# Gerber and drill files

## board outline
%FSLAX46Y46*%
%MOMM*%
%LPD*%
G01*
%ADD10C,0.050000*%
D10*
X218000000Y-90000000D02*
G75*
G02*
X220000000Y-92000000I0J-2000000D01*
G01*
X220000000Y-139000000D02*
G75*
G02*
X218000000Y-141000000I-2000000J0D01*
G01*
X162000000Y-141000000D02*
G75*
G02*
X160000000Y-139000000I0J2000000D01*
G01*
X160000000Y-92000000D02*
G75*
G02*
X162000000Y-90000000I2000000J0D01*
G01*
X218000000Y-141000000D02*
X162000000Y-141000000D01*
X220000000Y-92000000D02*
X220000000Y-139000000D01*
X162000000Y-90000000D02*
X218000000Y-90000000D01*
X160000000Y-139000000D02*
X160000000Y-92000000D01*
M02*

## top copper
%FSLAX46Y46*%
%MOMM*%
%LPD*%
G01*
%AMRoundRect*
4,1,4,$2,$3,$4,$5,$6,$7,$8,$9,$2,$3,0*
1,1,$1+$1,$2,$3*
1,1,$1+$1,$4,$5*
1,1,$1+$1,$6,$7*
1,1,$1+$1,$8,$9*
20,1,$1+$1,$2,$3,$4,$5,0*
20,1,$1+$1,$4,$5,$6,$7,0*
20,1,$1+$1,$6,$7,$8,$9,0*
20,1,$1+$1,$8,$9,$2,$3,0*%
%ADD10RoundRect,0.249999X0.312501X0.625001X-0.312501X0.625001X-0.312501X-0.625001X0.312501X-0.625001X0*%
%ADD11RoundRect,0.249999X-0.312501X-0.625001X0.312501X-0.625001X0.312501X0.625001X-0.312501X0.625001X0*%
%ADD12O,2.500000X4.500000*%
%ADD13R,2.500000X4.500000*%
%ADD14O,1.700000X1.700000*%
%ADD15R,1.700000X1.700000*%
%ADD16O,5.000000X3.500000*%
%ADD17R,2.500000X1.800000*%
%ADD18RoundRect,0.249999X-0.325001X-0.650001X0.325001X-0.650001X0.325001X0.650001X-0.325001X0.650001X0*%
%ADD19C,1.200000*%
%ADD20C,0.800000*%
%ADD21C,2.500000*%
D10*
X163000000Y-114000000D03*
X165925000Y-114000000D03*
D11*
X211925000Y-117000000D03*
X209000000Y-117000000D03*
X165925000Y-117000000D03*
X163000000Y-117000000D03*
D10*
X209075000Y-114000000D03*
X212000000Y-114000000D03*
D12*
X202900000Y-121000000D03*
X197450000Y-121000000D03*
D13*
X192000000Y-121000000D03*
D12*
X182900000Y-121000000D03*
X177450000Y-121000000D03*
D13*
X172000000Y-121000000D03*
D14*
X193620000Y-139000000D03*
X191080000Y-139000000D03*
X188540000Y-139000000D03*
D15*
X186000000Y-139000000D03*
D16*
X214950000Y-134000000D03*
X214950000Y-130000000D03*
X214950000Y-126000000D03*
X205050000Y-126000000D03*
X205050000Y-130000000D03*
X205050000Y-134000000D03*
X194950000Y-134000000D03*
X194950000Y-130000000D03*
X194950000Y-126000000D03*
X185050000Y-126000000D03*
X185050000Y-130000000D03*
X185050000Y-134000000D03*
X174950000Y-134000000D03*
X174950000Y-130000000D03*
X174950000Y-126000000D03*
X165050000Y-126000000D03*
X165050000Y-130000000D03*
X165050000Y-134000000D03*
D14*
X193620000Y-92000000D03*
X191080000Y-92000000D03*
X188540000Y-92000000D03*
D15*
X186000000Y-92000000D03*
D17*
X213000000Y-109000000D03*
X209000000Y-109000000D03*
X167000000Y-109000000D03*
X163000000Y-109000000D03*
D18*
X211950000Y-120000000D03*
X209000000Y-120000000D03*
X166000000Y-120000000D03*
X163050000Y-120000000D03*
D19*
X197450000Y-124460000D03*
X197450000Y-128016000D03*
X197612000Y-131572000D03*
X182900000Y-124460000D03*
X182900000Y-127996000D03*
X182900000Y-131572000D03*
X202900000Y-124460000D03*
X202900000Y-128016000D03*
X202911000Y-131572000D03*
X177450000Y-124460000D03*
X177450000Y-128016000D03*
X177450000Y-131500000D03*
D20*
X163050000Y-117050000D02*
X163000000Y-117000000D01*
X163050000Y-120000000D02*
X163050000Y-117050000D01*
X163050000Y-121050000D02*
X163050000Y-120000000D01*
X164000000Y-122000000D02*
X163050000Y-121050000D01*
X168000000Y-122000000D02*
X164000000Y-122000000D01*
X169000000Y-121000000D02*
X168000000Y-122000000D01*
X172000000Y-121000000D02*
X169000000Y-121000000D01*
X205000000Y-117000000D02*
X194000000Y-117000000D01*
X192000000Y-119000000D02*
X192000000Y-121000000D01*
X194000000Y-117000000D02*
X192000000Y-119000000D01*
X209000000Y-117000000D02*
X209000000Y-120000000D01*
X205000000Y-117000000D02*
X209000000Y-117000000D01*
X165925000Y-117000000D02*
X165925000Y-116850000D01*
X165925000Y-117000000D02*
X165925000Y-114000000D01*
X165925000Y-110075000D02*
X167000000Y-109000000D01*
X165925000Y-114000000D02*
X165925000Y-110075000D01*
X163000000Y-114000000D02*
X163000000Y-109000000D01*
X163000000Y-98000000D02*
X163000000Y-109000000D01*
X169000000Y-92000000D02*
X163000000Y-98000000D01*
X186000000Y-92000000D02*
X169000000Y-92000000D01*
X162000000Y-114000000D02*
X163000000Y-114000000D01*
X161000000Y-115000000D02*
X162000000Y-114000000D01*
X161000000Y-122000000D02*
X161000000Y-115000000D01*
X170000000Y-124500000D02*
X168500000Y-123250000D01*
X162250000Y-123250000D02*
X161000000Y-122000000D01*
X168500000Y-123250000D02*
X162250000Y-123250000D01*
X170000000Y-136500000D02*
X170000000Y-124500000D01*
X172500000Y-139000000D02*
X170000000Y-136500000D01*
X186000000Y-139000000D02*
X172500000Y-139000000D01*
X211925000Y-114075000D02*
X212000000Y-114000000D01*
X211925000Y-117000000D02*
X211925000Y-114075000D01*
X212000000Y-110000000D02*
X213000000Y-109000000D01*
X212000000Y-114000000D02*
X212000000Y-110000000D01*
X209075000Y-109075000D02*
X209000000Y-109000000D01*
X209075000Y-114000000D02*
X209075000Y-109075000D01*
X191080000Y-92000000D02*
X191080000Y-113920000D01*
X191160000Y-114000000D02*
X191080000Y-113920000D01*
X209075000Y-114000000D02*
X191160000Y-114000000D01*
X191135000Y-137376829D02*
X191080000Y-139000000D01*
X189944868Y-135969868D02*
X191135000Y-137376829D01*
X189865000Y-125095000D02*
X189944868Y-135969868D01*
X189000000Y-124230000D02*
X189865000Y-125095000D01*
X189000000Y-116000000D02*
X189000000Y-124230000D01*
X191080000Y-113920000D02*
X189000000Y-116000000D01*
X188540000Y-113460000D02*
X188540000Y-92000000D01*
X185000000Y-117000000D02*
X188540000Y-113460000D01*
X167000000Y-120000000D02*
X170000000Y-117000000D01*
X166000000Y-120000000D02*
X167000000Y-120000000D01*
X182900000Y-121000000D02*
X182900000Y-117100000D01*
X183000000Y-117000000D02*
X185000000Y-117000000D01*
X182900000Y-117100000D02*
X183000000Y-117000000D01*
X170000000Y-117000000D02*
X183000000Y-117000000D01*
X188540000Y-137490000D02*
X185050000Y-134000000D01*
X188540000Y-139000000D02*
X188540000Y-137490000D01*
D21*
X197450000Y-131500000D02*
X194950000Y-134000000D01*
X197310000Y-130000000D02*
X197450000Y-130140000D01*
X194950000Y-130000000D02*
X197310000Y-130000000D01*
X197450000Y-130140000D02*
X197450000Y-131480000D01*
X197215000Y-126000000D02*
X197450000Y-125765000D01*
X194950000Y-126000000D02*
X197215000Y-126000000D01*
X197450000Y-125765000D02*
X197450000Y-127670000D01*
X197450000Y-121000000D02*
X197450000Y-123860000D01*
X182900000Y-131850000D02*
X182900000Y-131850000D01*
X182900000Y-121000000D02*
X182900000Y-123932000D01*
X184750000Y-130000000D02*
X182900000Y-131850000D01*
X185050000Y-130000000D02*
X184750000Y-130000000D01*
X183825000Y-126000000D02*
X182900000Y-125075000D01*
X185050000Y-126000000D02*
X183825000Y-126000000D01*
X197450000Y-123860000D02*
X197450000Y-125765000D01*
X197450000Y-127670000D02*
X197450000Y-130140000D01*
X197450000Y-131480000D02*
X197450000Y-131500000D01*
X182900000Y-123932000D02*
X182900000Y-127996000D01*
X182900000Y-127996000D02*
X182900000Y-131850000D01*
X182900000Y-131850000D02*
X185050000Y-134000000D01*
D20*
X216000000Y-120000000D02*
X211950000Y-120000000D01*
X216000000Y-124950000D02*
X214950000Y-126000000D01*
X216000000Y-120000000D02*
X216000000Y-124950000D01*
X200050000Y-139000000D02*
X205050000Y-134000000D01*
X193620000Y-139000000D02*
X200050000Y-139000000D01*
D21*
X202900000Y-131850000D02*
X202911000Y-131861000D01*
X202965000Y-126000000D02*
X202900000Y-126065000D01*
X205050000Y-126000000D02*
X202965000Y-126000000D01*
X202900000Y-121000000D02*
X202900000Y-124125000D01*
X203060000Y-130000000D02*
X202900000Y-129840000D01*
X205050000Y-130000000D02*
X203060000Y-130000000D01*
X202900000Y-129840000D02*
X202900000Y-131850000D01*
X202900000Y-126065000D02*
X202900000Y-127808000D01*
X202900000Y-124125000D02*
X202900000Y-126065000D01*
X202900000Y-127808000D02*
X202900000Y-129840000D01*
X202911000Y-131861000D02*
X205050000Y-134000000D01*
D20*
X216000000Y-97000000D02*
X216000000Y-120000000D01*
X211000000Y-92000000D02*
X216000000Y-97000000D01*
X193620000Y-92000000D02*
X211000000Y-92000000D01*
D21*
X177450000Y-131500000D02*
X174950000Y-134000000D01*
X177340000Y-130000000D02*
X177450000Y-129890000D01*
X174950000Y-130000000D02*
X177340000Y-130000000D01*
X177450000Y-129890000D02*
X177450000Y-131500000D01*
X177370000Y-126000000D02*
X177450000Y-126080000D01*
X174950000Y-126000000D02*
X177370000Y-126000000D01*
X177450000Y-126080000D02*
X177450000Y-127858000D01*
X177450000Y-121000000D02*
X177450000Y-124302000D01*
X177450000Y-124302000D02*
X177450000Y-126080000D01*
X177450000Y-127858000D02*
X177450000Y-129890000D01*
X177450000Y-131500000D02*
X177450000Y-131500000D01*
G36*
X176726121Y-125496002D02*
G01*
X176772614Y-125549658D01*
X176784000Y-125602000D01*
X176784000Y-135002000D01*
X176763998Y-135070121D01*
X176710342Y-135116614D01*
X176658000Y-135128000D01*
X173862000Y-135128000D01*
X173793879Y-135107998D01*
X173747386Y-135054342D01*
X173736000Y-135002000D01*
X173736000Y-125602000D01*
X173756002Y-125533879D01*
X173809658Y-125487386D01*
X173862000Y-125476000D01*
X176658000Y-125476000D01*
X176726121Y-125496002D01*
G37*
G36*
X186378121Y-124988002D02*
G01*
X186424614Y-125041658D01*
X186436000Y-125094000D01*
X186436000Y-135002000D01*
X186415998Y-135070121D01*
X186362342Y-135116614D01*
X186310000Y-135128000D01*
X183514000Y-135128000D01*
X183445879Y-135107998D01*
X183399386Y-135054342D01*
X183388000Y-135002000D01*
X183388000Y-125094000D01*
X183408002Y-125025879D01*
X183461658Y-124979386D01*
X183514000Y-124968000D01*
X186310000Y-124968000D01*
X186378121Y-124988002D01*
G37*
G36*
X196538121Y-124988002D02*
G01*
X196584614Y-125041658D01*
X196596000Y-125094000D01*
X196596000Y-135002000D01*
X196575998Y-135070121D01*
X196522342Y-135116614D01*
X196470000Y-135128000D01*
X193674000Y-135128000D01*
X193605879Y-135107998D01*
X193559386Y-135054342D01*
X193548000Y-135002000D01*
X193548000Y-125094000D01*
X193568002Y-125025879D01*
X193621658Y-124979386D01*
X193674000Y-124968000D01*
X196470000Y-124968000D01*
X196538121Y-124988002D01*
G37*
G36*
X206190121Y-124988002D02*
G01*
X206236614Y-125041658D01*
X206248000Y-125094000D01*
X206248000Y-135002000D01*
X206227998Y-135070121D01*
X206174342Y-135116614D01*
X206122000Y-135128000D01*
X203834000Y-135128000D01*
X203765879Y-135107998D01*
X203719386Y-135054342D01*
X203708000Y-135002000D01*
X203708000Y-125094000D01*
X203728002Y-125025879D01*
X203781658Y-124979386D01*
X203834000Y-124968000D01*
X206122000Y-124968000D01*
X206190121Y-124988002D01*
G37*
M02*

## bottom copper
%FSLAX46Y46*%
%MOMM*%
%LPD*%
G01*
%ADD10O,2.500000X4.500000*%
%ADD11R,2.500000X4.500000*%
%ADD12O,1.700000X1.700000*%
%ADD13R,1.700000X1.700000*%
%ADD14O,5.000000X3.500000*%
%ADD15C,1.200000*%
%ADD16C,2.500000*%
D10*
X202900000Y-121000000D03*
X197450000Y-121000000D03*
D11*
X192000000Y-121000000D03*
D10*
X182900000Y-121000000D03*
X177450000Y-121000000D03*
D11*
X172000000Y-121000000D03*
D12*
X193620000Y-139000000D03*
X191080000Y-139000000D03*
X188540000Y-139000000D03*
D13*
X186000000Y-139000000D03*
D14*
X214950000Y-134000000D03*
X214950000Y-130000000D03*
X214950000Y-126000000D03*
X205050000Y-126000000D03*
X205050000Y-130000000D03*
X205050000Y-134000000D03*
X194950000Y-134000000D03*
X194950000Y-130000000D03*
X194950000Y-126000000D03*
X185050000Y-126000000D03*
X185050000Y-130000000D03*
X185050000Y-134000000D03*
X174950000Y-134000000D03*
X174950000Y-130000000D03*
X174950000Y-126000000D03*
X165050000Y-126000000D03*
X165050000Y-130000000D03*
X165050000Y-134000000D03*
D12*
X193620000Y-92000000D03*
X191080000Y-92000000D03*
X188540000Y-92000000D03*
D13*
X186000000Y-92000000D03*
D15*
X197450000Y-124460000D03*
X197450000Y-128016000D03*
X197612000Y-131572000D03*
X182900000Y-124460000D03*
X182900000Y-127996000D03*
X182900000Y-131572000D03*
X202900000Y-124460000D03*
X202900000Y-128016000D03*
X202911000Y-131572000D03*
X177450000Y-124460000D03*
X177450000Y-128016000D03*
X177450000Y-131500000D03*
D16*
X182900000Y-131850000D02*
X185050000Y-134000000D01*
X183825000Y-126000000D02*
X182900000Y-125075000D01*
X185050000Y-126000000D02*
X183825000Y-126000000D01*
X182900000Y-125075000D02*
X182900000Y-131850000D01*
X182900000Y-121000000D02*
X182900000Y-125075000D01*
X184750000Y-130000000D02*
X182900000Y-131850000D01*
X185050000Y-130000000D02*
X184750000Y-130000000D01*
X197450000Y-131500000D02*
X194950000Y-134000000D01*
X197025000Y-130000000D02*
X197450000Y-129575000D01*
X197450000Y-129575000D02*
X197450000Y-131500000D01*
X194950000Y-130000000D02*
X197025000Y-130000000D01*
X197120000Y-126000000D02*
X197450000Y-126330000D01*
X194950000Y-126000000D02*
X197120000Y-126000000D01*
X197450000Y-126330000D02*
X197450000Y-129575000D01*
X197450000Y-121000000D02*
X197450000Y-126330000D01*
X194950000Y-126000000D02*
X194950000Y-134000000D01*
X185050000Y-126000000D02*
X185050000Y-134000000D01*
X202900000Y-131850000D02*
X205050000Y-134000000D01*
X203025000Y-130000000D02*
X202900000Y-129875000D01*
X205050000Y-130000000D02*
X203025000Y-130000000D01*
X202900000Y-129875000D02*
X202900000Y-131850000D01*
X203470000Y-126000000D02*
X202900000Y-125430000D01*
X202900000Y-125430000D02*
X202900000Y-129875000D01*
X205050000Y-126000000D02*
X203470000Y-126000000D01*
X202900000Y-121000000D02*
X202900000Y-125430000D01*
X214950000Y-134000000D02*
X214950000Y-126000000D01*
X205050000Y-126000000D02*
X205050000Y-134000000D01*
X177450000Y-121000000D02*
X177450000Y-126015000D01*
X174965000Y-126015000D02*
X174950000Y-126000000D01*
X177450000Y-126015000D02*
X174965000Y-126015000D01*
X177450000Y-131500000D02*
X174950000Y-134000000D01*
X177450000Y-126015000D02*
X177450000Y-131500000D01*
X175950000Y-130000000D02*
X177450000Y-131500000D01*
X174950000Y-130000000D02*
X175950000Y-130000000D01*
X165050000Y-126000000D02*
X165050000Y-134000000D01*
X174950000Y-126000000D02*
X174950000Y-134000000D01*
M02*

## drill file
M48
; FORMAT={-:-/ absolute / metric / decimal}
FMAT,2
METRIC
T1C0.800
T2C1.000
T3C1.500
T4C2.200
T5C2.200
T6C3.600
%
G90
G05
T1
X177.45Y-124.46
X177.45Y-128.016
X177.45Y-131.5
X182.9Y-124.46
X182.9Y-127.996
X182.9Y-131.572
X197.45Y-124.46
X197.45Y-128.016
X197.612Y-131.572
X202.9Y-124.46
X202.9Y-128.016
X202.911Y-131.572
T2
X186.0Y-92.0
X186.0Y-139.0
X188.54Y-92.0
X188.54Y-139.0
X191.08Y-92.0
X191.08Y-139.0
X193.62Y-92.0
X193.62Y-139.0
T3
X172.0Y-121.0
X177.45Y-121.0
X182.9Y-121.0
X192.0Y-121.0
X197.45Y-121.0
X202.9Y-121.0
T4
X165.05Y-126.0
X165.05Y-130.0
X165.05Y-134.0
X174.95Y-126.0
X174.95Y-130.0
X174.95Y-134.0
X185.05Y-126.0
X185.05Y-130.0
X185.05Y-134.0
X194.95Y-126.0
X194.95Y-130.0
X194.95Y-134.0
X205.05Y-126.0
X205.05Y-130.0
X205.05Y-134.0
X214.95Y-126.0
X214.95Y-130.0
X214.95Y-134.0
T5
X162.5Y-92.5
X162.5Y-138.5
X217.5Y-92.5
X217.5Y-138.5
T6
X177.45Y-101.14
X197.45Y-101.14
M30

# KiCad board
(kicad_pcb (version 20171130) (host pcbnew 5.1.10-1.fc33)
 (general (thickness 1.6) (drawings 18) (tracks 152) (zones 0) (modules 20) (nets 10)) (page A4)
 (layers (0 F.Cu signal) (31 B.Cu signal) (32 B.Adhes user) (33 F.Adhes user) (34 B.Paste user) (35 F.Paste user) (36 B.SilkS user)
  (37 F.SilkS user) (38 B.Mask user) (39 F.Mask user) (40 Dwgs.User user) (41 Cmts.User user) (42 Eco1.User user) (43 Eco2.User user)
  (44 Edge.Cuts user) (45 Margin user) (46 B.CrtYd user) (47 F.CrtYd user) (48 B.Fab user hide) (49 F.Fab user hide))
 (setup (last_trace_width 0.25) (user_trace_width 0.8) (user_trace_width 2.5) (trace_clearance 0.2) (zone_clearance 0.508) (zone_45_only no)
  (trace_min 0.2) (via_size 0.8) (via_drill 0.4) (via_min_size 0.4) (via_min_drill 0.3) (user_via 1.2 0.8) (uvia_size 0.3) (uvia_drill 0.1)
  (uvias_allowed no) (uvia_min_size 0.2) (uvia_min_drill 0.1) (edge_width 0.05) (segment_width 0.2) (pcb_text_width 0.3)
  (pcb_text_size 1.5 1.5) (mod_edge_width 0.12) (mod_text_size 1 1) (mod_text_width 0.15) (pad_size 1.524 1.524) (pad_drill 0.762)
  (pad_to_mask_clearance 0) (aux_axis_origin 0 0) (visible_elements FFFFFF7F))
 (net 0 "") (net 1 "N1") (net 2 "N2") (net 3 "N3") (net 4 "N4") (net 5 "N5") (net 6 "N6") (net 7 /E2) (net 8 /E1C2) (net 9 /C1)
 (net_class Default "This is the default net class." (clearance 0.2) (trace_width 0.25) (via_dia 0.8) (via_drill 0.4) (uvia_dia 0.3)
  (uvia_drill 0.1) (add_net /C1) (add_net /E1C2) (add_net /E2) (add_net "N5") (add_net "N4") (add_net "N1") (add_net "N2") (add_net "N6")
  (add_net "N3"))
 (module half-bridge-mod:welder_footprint (layer F.Cu) (at 178.5 110.7)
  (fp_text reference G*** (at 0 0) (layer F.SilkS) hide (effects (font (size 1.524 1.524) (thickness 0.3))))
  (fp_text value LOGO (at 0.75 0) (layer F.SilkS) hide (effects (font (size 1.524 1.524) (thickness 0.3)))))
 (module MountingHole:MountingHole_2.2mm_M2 (layer F.Cu) (at 162.5 138.5)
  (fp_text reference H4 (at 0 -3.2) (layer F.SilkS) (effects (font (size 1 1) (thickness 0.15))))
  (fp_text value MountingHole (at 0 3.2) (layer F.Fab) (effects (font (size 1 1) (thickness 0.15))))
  (pad 1 np_thru_hole circle (at 0 0) (size 2.2 2.2) (drill 2.2) (layers *.Cu *.Mask)))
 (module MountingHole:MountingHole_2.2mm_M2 (layer F.Cu) (at 217.5 138.5)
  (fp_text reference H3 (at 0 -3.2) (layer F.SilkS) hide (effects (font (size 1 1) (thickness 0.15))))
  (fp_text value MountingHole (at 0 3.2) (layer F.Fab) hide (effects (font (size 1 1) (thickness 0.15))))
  (pad 1 np_thru_hole circle (at 0 0) (size 2.2 2.2) (drill 2.2) (layers *.Cu *.Mask)))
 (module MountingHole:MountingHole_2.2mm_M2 (layer F.Cu) (at 162.5 92.5)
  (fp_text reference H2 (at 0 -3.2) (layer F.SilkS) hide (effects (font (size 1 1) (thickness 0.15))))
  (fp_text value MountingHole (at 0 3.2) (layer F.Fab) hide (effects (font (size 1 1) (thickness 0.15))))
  (pad 1 np_thru_hole circle (at 0 0) (size 2.2 2.2) (drill 2.2) (layers *.Cu *.Mask)))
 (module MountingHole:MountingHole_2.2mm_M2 (layer F.Cu) (at 217.5 92.5)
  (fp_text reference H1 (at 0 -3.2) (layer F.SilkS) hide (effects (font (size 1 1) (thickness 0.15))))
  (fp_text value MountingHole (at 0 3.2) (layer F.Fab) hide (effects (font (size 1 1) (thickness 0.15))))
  (pad 1 np_thru_hole circle (at 0 0) (size 2.2 2.2) (drill 2.2) (layers *.Cu *.Mask)))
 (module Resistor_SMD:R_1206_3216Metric (layer F.Cu) (at 164.4625 114 180)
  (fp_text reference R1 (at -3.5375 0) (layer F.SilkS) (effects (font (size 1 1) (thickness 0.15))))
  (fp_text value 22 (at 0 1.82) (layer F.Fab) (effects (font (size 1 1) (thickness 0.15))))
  (pad 2 smd roundrect (at 1.4625 0 180) (size 1.125 1.75) (layers F.Cu F.Paste F.Mask) (roundrect_rratio 0.2222213333333333) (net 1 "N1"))
  (pad 1 smd roundrect (at -1.4625 0 180) (size 1.125 1.75) (layers F.Cu F.Paste F.Mask) (roundrect_rratio 0.2222213333333333) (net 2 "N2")))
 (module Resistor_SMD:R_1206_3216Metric (layer F.Cu) (at 210.4625 117)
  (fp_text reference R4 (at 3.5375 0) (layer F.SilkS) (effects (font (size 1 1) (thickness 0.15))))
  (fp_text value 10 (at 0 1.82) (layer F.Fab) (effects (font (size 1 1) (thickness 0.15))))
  (pad 2 smd roundrect (at 1.4625 0) (size 1.125 1.75) (layers F.Cu F.Paste F.Mask) (roundrect_rratio 0.2222213333333333) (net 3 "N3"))
  (pad 1 smd roundrect (at -1.4625 0) (size 1.125 1.75) (layers F.Cu F.Paste F.Mask) (roundrect_rratio 0.2222213333333333) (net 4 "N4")))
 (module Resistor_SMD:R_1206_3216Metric (layer F.Cu) (at 164.4625 117)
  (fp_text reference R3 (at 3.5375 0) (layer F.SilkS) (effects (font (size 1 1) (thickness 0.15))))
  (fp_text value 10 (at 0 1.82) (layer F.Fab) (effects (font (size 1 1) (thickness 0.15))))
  (pad 2 smd roundrect (at 1.4625 0) (size 1.125 1.75) (layers F.Cu F.Paste F.Mask) (roundrect_rratio 0.2222213333333333) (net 2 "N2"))
  (pad 1 smd roundrect (at -1.4625 0) (size 1.125 1.75) (layers F.Cu F.Paste F.Mask) (roundrect_rratio 0.2222213333333333) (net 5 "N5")))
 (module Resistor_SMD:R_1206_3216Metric (layer F.Cu) (at 210.5375 114 180)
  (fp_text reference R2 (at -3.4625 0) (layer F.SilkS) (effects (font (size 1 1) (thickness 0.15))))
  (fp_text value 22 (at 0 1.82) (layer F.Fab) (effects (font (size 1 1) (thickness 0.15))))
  (pad 2 smd roundrect (at 1.4625 0 180) (size 1.125 1.75) (layers F.Cu F.Paste F.Mask) (roundrect_rratio 0.2222213333333333) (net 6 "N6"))
  (pad 1 smd roundrect (at -1.4625 0 180) (size 1.125 1.75) (layers F.Cu F.Paste F.Mask) (roundrect_rratio 0.2222213333333333) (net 3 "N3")))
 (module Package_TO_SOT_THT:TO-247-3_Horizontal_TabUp (layer B.Cu) (at 192 121)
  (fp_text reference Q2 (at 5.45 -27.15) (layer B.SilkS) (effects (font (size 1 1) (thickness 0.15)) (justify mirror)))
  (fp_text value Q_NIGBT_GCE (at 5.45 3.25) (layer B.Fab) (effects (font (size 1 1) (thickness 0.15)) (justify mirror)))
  (pad 3 thru_hole oval (at 10.9 0) (size 2.5 4.5) (drill 1.5) (layers *.Cu *.Mask) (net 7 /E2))
  (pad 2 thru_hole oval (at 5.45 0) (size 2.5 4.5) (drill 1.5) (layers *.Cu *.Mask) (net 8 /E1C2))
  (pad 1 thru_hole rect (at 0 0) (size 2.5 4.5) (drill 1.5) (layers *.Cu *.Mask) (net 4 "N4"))
  (pad "" np_thru_hole oval (at 5.45 -19.86) (size 3.6 3.6) (drill 3.6) (layers *.Cu *.Mask)))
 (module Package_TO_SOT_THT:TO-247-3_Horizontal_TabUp (layer B.Cu) (at 172 121)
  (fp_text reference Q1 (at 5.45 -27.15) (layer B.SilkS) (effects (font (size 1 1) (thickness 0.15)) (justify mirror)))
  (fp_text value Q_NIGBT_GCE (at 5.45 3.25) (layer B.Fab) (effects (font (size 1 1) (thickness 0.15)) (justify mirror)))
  (pad 3 thru_hole oval (at 10.9 0) (size 2.5 4.5) (drill 1.5) (layers *.Cu *.Mask) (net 8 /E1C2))
  (pad 2 thru_hole oval (at 5.45 0) (size 2.5 4.5) (drill 1.5) (layers *.Cu *.Mask) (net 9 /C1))
  (pad 1 thru_hole rect (at 0 0) (size 2.5 4.5) (drill 1.5) (layers *.Cu *.Mask) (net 5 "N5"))
  (pad "" np_thru_hole oval (at 5.45 -19.86) (size 3.6 3.6) (drill 3.6) (layers *.Cu *.Mask)))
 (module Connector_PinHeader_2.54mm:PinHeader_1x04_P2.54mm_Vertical (layer F.Cu) (at 186 139 90)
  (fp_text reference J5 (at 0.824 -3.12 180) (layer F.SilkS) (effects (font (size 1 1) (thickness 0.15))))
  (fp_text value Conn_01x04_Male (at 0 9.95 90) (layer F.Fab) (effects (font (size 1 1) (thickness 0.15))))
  (pad 4 thru_hole oval (at 0 7.62 90) (size 1.7 1.7) (drill 1) (layers *.Cu *.Mask) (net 7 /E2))
  (pad 3 thru_hole oval (at 0 5.08 90) (size 1.7 1.7) (drill 1) (layers *.Cu *.Mask) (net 6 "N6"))
  (pad 2 thru_hole oval (at 0 2.54 90) (size 1.7 1.7) (drill 1) (layers *.Cu *.Mask) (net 8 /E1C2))
  (pad 1 thru_hole rect (at 0 0 90) (size 1.7 1.7) (drill 1) (layers *.Cu *.Mask) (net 1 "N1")))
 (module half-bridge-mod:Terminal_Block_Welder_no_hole (layer F.Cu) (at 210 130 90)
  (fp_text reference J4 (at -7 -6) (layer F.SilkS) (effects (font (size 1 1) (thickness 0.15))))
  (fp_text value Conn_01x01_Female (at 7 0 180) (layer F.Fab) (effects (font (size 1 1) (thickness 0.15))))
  (pad 1 thru_hole oval (at -4 4.95 180) (size 5 3.5) (drill 2.2) (layers *.Cu *.Mask) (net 7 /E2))
  (pad 1 thru_hole oval (at 0 4.95 180) (size 5 3.5) (drill 2.2) (layers *.Cu *.Mask) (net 7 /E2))
  (pad 1 thru_hole oval (at 4 4.95 180) (size 5 3.5) (drill 2.2) (layers *.Cu *.Mask) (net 7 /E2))
  (pad 1 thru_hole oval (at 4 -4.95 180) (size 5 3.5) (drill 2.2) (layers *.Cu *.Mask) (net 7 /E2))
  (pad 1 thru_hole oval (at 0 -4.95 180) (size 5 3.5) (drill 2.2) (layers *.Cu *.Mask) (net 7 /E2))
  (pad 1 thru_hole oval (at -4 -4.95 180) (size 5 3.5) (drill 2.2) (layers *.Cu *.Mask) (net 7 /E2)))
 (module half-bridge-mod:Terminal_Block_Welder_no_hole (layer F.Cu) (at 190 130 90)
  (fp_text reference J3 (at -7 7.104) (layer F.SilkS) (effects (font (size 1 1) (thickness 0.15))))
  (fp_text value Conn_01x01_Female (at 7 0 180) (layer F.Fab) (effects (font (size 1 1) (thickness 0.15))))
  (pad 1 thru_hole oval (at -4 4.95 180) (size 5 3.5) (drill 2.2) (layers *.Cu *.Mask) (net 8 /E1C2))
  (pad 1 thru_hole oval (at 0 4.95 180) (size 5 3.5) (drill 2.2) (layers *.Cu *.Mask) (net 8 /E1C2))
  (pad 1 thru_hole oval (at 4 4.95 180) (size 5 3.5) (drill 2.2) (layers *.Cu *.Mask) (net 8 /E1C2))
  (pad 1 thru_hole oval (at 4 -4.95 180) (size 5 3.5) (drill 2.2) (layers *.Cu *.Mask) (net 8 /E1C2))
  (pad 1 thru_hole oval (at 0 -4.95 180) (size 5 3.5) (drill 2.2) (layers *.Cu *.Mask) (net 8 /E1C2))
  (pad 1 thru_hole oval (at -4 -4.95 180) (size 5 3.5) (drill 2.2) (layers *.Cu *.Mask) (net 8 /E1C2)))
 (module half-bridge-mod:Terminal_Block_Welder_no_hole (layer F.Cu) (at 170 130 90)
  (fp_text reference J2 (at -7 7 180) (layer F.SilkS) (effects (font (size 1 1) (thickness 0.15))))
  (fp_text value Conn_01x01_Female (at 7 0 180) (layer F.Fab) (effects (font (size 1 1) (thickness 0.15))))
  (pad 1 thru_hole oval (at -4 4.95 180) (size 5 3.5) (drill 2.2) (layers *.Cu *.Mask) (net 9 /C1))
  (pad 1 thru_hole oval (at 0 4.95 180) (size 5 3.5) (drill 2.2) (layers *.Cu *.Mask) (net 9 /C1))
  (pad 1 thru_hole oval (at 4 4.95 180) (size 5 3.5) (drill 2.2) (layers *.Cu *.Mask) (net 9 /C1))
  (pad 1 thru_hole oval (at 4 -4.95 180) (size 5 3.5) (drill 2.2) (layers *.Cu *.Mask) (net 9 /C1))
  (pad 1 thru_hole oval (at 0 -4.95 180) (size 5 3.5) (drill 2.2) (layers *.Cu *.Mask) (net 9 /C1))
  (pad 1 thru_hole oval (at -4 -4.95 180) (size 5 3.5) (drill 2.2) (layers *.Cu *.Mask) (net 9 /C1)))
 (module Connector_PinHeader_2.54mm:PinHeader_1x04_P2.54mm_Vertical (layer F.Cu) (at 186 92 90)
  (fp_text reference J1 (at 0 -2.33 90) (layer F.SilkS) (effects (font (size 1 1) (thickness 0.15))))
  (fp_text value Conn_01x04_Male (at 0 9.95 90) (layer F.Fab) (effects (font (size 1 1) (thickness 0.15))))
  (pad 4 thru_hole oval (at 0 7.62 90) (size 1.7 1.7) (drill 1) (layers *.Cu *.Mask) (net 7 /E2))
  (pad 3 thru_hole oval (at 0 5.08 90) (size 1.7 1.7) (drill 1) (layers *.Cu *.Mask) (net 6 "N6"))
  (pad 2 thru_hole oval (at 0 2.54 90) (size 1.7 1.7) (drill 1) (layers *.Cu *.Mask) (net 8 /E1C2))
  (pad 1 thru_hole rect (at 0 0 90) (size 1.7 1.7) (drill 1) (layers *.Cu *.Mask) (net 1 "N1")))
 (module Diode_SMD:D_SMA (layer F.Cu) (at 211 109)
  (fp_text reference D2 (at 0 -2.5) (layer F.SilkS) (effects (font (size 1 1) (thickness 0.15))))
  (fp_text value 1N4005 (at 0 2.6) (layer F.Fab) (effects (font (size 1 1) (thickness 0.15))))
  (pad 2 smd rect (at 2 0) (size 2.5 1.8) (layers F.Cu F.Paste F.Mask) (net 3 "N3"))
  (pad 1 smd rect (at -2 0) (size 2.5 1.8) (layers F.Cu F.Paste F.Mask) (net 6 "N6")))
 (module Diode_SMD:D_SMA (layer F.Cu) (at 165 109)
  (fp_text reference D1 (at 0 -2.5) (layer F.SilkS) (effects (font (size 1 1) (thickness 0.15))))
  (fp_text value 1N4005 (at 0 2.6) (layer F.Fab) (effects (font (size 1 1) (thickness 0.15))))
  (pad 2 smd rect (at 2 0) (size 2.5 1.8) (layers F.Cu F.Paste F.Mask) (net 2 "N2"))
  (pad 1 smd rect (at -2 0) (size 2.5 1.8) (layers F.Cu F.Paste F.Mask) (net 1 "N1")))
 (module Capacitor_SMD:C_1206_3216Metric (layer F.Cu) (at 210.475 120)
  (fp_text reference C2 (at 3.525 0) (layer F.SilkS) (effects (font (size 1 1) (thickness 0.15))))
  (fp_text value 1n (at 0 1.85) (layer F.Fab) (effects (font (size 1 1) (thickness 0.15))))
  (pad 2 smd roundrect (at 1.475 0) (size 1.15 1.8) (layers F.Cu F.Paste F.Mask) (roundrect_rratio 0.2173904347826087) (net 7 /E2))
  (pad 1 smd roundrect (at -1.475 0) (size 1.15 1.8) (layers F.Cu F.Paste F.Mask) (roundrect_rratio 0.2173904347826087) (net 4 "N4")))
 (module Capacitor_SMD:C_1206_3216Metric (layer F.Cu) (at 164.525 120)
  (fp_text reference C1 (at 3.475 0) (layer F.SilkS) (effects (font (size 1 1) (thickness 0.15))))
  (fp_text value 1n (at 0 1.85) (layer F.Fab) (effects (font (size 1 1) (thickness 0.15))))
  (pad 2 smd roundrect (at 1.475 0) (size 1.15 1.8) (layers F.Cu F.Paste F.Mask) (roundrect_rratio 0.2173904347826087) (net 8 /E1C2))
  (pad 1 smd roundrect (at -1.475 0) (size 1.15 1.8) (layers F.Cu F.Paste F.Mask) (roundrect_rratio 0.2173904347826087) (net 5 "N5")))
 (gr_arc (start 218 92) (end 220 92) (angle -90) (layer Edge.Cuts) (width 0.05))
 (gr_arc (start 218 139) (end 218 141) (angle -90) (layer Edge.Cuts) (width 0.05))
 (gr_arc (start 162 139) (end 160 139) (angle -90) (layer Edge.Cuts) (width 0.05))
 (gr_arc (start 162 92) (end 162 90) (angle -90) (layer Edge.Cuts) (width 0.05))
 (gr_line (start 218 141) (end 162 141) (layer Edge.Cuts) (width 0.05))
 (gr_line (start 220 92) (end 220 139) (layer Edge.Cuts) (width 0.05))
 (gr_line (start 162 90) (end 218 90) (layer Edge.Cuts) (width 0.05))
 (gr_line (start 160 139) (end 160 92) (layer Edge.Cuts) (width 0.05))
 (segment (start 163.05 117.05) (end 163 117) (width 0.8) (layer F.Cu) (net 5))
 (segment (start 163.05 120) (end 163.05 117.05) (width 0.8) (layer F.Cu) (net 5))
 (segment (start 163.05 121.05) (end 163.05 120) (width 0.8) (layer F.Cu) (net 5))
 (segment (start 164 122) (end 163.05 121.05) (width 0.8) (layer F.Cu) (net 5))
 (segment (start 168 122) (end 164 122) (width 0.8) (layer F.Cu) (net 5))
 (segment (start 169 121) (end 168 122) (width 0.8) (layer F.Cu) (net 5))
 (segment (start 172 121) (end 169 121) (width 0.8) (layer F.Cu) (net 5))
 (segment (start 205 117) (end 194 117) (width 0.8) (layer F.Cu) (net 4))
 (segment (start 192 119) (end 192 121) (width 0.8) (layer F.Cu) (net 4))
 (segment (start 194 117) (end 192 119) (width 0.8) (layer F.Cu) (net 4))
 (segment (start 209 117) (end 209 120) (width 0.8) (layer F.Cu) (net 4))
 (segment (start 205 117) (end 209 117) (width 0.8) (layer F.Cu) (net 4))
 (segment (start 165.925 117) (end 165.925 116.85) (width 0.8) (layer F.Cu) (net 2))
 (segment (start 165.925 117) (end 165.925 114) (width 0.8) (layer F.Cu) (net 2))
 (segment (start 165.925 110.075) (end 167 109) (width 0.8) (layer F.Cu) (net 2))
 (segment (start 165.925 114) (end 165.925 110.075) (width 0.8) (layer F.Cu) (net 2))
 (segment (start 163 114) (end 163 109) (width 0.8) (layer F.Cu) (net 1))
 (segment (start 163 98) (end 163 109) (width 0.8) (layer F.Cu) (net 1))
 (segment (start 169 92) (end 163 98) (width 0.8) (layer F.Cu) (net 1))
 (segment (start 186 92) (end 169 92) (width 0.8) (layer F.Cu) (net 1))
 (segment (start 162 114) (end 163 114) (width 0.8) (layer F.Cu) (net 1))
 (segment (start 161 115) (end 162 114) (width 0.8) (layer F.Cu) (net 1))
 (segment (start 161 122) (end 161 115) (width 0.8) (layer F.Cu) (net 1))
 (segment (start 170 124.5) (end 168.5 123.25) (width 0.8) (layer F.Cu) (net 1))
 (segment (start 162.25 123.25) (end 161 122) (width 0.8) (layer F.Cu) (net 1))
 (segment (start 168.5 123.25) (end 162.25 123.25) (width 0.8) (layer F.Cu) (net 1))
 (segment (start 170 136.5) (end 170 124.5) (width 0.8) (layer F.Cu) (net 1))
 (segment (start 172.5 139) (end 170 136.5) (width 0.8) (layer F.Cu) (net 1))
 (segment (start 186 139) (end 172.5 139) (width 0.8) (layer F.Cu) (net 1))
 (segment (start 211.925 114.075) (end 212 114) (width 0.8) (layer F.Cu) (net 3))
 (segment (start 211.925 117) (end 211.925 114.075) (width 0.8) (layer F.Cu) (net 3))
 (segment (start 212 110) (end 213 109) (width 0.8) (layer F.Cu) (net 3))
 (segment (start 212 114) (end 212 110) (width 0.8) (layer F.Cu) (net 3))
 (segment (start 209.075 109.075) (end 209 109) (width 0.8) (layer F.Cu) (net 6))
 (segment (start 209.075 114) (end 209.075 109.075) (width 0.8) (layer F.Cu) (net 6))
 (segment (start 191.08 92) (end 191.08 113.92) (width 0.8) (layer F.Cu) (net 6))
 (segment (start 191.16 114) (end 191.08 113.92) (width 0.8) (layer F.Cu) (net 6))
 (segment (start 209.075 114) (end 191.16 114) (width 0.8) (layer F.Cu) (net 6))
 (segment (start 191.135 137.376829) (end 191.08 139) (width 0.8) (layer F.Cu) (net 6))
 (segment (start 189.944868 135.969868) (end 191.135 137.376829) (width 0.8) (layer F.Cu) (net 6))
 (segment (start 189.865 125.095) (end 189.944868 135.969868) (width 0.8) (layer F.Cu) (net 6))
 (segment (start 189 124.23) (end 189.865 125.095) (width 0.8) (layer F.Cu) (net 6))
 (segment (start 189 116) (end 189 124.23) (width 0.8) (layer F.Cu) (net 6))
 (segment (start 191.08 113.92) (end 189 116) (width 0.8) (layer F.Cu) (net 6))
 (segment (start 188.54 113.46) (end 188.54 92) (width 0.8) (layer F.Cu) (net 8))
 (segment (start 185 117) (end 188.54 113.46) (width 0.8) (layer F.Cu) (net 8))
 (segment (start 167 120) (end 170 117) (width 0.8) (layer F.Cu) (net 8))
 (segment (start 166 120) (end 167 120) (width 0.8) (layer F.Cu) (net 8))
 (segment (start 182.9 121) (end 182.9 117.1) (width 0.8) (layer F.Cu) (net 8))
 (segment (start 183 117) (end 185 117) (width 0.8) (layer F.Cu) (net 8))
 (segment (start 182.9 117.1) (end 183 117) (width 0.8) (layer F.Cu) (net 8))
 (segment (start 170 117) (end 183 117) (width 0.8) (layer F.Cu) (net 8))
 (segment (start 188.54 137.49) (end 185.05 134) (width 0.8) (layer F.Cu) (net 8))
 (segment (start 188.54 139) (end 188.54 137.49) (width 0.8) (layer F.Cu) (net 8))
 (segment (start 182.9 131.85) (end 185.05 134) (width 2.5) (layer B.Cu) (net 8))
 (segment (start 183.825 126) (end 182.9 125.075) (width 2.5) (layer B.Cu) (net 8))
 (segment (start 185.05 126) (end 183.825 126) (width 2.5) (layer B.Cu) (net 8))
 (segment (start 182.9 125.075) (end 182.9 131.85) (width 2.5) (layer B.Cu) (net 8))
 (segment (start 182.9 121) (end 182.9 125.075) (width 2.5) (layer B.Cu) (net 8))
 (segment (start 184.75 130) (end 182.9 131.85) (width 2.5) (layer B.Cu) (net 8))
 (segment (start 185.05 130) (end 184.75 130) (width 2.5) (layer B.Cu) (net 8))
 (segment (start 197.45 131.5) (end 194.95 134) (width 2.5) (layer B.Cu) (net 8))
 (segment (start 197.025 130) (end 197.45 129.575) (width 2.5) (layer B.Cu) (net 8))
 (segment (start 197.45 129.575) (end 197.45 131.5) (width 2.5) (layer B.Cu) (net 8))
 (segment (start 194.95 130) (end 197.025 130) (width 2.5) (layer B.Cu) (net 8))
 (segment (start 197.12 126) (end 197.45 126.33) (width 2.5) (layer B.Cu) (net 8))
 (segment (start 194.95 126) (end 197.12 126) (width 2.5) (layer B.Cu) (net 8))
 (segment (start 197.45 126.33) (end 197.45 129.575) (width 2.5) (layer B.Cu) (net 8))
 (segment (start 197.45 121) (end 197.45 126.33) (width 2.5) (layer B.Cu) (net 8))
 (segment (start 197.45 131.5) (end 194.95 134) (width 2.5) (layer F.Cu) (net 8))
 (segment (start 197.31 130) (end 197.45 130.14) (width 2.5) (layer F.Cu) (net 8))
 (segment (start 194.95 130) (end 197.31 130) (width 2.5) (layer F.Cu) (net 8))
 (segment (start 197.45 130.14) (end 197.45 131.48) (width 2.5) (layer F.Cu) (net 8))
 (segment (start 197.215 126) (end 197.45 125.765) (width 2.5) (layer F.Cu) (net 8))
 (segment (start 194.95 126) (end 197.215 126) (width 2.5) (layer F.Cu) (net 8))
 (segment (start 197.45 125.765) (end 197.45 127.67) (width 2.5) (layer F.Cu) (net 8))
 (segment (start 197.45 121) (end 197.45 123.86) (width 2.5) (layer F.Cu) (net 8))
 (segment (start 182.9 131.85) (end 182.9 131.85) (width 2.5) (layer F.Cu) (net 8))
 (segment (start 182.9 121) (end 182.9 123.932) (width 2.5) (layer F.Cu) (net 8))
 (segment (start 184.75 130) (end 182.9 131.85) (width 2.5) (layer F.Cu) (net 8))
 (segment (start 185.05 130) (end 184.75 130) (width 2.5) (layer F.Cu) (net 8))
 (segment (start 183.825 126) (end 182.9 125.075) (width 2.5) (layer F.Cu) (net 8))
 (segment (start 185.05 126) (end 183.825 126) (width 2.5) (layer F.Cu) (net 8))
 (segment (start 194.95 126) (end 194.95 134) (width 2.5) (layer B.Cu) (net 8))
 (segment (start 185.05 126) (end 185.05 134) (width 2.5) (layer B.Cu) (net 8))
 (segment (start 197.45 123.86) (end 197.45 125.765) (width 2.5) (layer F.Cu) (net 8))
 (via (at 197.45 124.46) (size 1.2) (drill 0.8) (layers F.Cu B.Cu) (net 8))
 (segment (start 197.45 127.67) (end 197.45 130.14) (width 2.5) (layer F.Cu) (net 8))
 (via (at 197.45 128.016) (size 1.2) (drill 0.8) (layers F.Cu B.Cu) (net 8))
 (segment (start 197.45 131.48) (end 197.45 131.5) (width 2.5) (layer F.Cu) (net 8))
 (via (at 197.612 131.572) (size 1.2) (drill 0.8) (layers F.Cu B.Cu) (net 8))
 (segment (start 182.9 123.932) (end 182.9 127.996) (width 2.5) (layer F.Cu) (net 8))
 (via (at 182.9 124.46) (size 1.2) (drill 0.8) (layers F.Cu B.Cu) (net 8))
 (segment (start 182.9 127.996) (end 182.9 131.85) (width 2.5) (layer F.Cu) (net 8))
 (via (at 182.9 127.996) (size 1.2) (drill 0.8) (layers F.Cu B.Cu) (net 8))
 (segment (start 182.9 131.85) (end 185.05 134) (width 2.5) (layer F.Cu) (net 8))
 (via (at 182.9 131.572) (size 1.2) (drill 0.8) (layers F.Cu B.Cu) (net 8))
 (segment (start 216 120) (end 211.95 120) (width 0.8) (layer F.Cu) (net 7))
 (segment (start 216 124.95) (end 214.95 126) (width 0.8) (layer F.Cu) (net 7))
 (segment (start 216 120) (end 216 124.95) (width 0.8) (layer F.Cu) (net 7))
 (segment (start 200.05 139) (end 205.05 134) (width 0.8) (layer F.Cu) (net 7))
 (segment (start 193.62 139) (end 200.05 139) (width 0.8) (layer F.Cu) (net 7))
 (segment (start 202.9 131.85) (end 205.05 134) (width 2.5) (layer B.Cu) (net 7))
 (segment (start 203.025 130) (end 202.9 129.875) (width 2.5) (layer B.Cu) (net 7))
 (segment (start 205.05 130) (end 203.025 130) (width 2.5) (layer B.Cu) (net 7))
 (segment (start 202.9 129.875) (end 202.9 131.85) (width 2.5) (layer B.Cu) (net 7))
 (segment (start 203.47 126) (end 202.9 125.43) (width 2.5) (layer B.Cu) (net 7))
 (segment (start 202.9 125.43) (end 202.9 129.875) (width 2.5) (layer B.Cu) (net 7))
 (segment (start 205.05 126) (end 203.47 126) (width 2.5) (layer B.Cu) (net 7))
 (segment (start 202.9 121) (end 202.9 125.43) (width 2.5) (layer B.Cu) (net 7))
 (segment (start 202.9 131.85) (end 202.911 131.861) (width 2.5) (layer F.Cu) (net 7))
 (segment (start 202.965 126) (end 202.9 126.065) (width 2.5) (layer F.Cu) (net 7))
 (segment (start 205.05 126) (end 202.965 126) (width 2.5) (layer F.Cu) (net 7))
 (segment (start 202.9 121) (end 202.9 124.125) (width 2.5) (layer F.Cu) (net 7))
 (segment (start 203.06 130) (end 202.9 129.84) (width 2.5) (layer F.Cu) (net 7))
 (segment (start 205.05 130) (end 203.06 130) (width 2.5) (layer F.Cu) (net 7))
 (segment (start 202.9 129.84) (end 202.9 131.85) (width 2.5) (layer F.Cu) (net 7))
 (segment (start 202.9 126.065) (end 202.9 127.808) (width 2.5) (layer F.Cu) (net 7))
 (segment (start 214.95 134) (end 214.95 126) (width 2.5) (layer B.Cu) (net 7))
 (segment (start 205.05 126) (end 205.05 134) (width 2.5) (layer B.Cu) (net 7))
 (segment (start 202.9 124.125) (end 202.9 126.065) (width 2.5) (layer F.Cu) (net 7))
 (via (at 202.9 124.46) (size 1.2) (drill 0.8) (layers F.Cu B.Cu) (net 7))
 (segment (start 202.9 127.808) (end 202.9 129.84) (width 2.5) (layer F.Cu) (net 7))
 (via (at 202.9 128.016) (size 1.2) (drill 0.8) (layers F.Cu B.Cu) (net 7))
 (segment (start 202.911 131.861) (end 205.05 134) (width 2.5) (layer F.Cu) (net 7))
 (via (at 202.911 131.572) (size 1.2) (drill 0.8) (layers F.Cu B.Cu) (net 7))
 (segment (start 216 97) (end 216 120) (width 0.8) (layer F.Cu) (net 7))
 (segment (start 211 92) (end 216 97) (width 0.8) (layer F.Cu) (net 7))
 (segment (start 193.62 92) (end 211 92) (width 0.8) (layer F.Cu) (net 7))
 (segment (start 177.45 121) (end 177.45 126.015) (width 2.5) (layer B.Cu) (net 9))
 (segment (start 174.965 126.015) (end 174.95 126) (width 2.5) (layer B.Cu) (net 9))
 (segment (start 177.45 126.015) (end 174.965 126.015) (width 2.5) (layer B.Cu) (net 9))
 (segment (start 177.45 131.5) (end 174.95 134) (width 2.5) (layer B.Cu) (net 9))
 (segment (start 177.45 126.015) (end 177.45 131.5) (width 2.5) (layer B.Cu) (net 9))
 (segment (start 175.95 130) (end 177.45 131.5) (width 2.5) (layer B.Cu) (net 9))
 (segment (start 174.95 130) (end 175.95 130) (width 2.5) (layer B.Cu) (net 9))
 (segment (start 165.05 126) (end 165.05 134) (width 2.5) (layer B.Cu) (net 9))
 (segment (start 177.45 131.5) (end 174.95 134) (width 2.5) (layer F.Cu) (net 9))
 (segment (start 177.34 130) (end 177.45 129.89) (width 2.5) (layer F.Cu) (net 9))
 (segment (start 174.95 130) (end 177.34 130) (width 2.5) (layer F.Cu) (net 9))
 (segment (start 177.45 129.89) (end 177.45 131.5) (width 2.5) (layer F.Cu) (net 9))
 (segment (start 177.37 126) (end 177.45 126.08) (width 2.5) (layer F.Cu) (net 9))
 (segment (start 174.95 126) (end 177.37 126) (width 2.5) (layer F.Cu) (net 9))
 (segment (start 177.45 126.08) (end 177.45 127.858) (width 2.5) (layer F.Cu) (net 9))
 (segment (start 177.45 121) (end 177.45 124.302) (width 2.5) (layer F.Cu) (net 9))
 (segment (start 174.95 126) (end 174.95 134) (width 2.5) (layer B.Cu) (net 9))
 (segment (start 177.45 124.302) (end 177.45 126.08) (width 2.5) (layer F.Cu) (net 9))
 (via (at 177.45 124.46) (size 1.2) (drill 0.8) (layers F.Cu B.Cu) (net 9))
 (segment (start 177.45 127.858) (end 177.45 129.89) (width 2.5) (layer F.Cu) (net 9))
 (via (at 177.45 128.016) (size 1.2) (drill 0.8) (layers F.Cu B.Cu) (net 9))
 (segment (start 177.45 131.5) (end 177.45 131.5) (width 2.5) (layer F.Cu) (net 9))
 (via (at 177.45 131.5) (size 1.2) (drill 0.8) (layers F.Cu B.Cu) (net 9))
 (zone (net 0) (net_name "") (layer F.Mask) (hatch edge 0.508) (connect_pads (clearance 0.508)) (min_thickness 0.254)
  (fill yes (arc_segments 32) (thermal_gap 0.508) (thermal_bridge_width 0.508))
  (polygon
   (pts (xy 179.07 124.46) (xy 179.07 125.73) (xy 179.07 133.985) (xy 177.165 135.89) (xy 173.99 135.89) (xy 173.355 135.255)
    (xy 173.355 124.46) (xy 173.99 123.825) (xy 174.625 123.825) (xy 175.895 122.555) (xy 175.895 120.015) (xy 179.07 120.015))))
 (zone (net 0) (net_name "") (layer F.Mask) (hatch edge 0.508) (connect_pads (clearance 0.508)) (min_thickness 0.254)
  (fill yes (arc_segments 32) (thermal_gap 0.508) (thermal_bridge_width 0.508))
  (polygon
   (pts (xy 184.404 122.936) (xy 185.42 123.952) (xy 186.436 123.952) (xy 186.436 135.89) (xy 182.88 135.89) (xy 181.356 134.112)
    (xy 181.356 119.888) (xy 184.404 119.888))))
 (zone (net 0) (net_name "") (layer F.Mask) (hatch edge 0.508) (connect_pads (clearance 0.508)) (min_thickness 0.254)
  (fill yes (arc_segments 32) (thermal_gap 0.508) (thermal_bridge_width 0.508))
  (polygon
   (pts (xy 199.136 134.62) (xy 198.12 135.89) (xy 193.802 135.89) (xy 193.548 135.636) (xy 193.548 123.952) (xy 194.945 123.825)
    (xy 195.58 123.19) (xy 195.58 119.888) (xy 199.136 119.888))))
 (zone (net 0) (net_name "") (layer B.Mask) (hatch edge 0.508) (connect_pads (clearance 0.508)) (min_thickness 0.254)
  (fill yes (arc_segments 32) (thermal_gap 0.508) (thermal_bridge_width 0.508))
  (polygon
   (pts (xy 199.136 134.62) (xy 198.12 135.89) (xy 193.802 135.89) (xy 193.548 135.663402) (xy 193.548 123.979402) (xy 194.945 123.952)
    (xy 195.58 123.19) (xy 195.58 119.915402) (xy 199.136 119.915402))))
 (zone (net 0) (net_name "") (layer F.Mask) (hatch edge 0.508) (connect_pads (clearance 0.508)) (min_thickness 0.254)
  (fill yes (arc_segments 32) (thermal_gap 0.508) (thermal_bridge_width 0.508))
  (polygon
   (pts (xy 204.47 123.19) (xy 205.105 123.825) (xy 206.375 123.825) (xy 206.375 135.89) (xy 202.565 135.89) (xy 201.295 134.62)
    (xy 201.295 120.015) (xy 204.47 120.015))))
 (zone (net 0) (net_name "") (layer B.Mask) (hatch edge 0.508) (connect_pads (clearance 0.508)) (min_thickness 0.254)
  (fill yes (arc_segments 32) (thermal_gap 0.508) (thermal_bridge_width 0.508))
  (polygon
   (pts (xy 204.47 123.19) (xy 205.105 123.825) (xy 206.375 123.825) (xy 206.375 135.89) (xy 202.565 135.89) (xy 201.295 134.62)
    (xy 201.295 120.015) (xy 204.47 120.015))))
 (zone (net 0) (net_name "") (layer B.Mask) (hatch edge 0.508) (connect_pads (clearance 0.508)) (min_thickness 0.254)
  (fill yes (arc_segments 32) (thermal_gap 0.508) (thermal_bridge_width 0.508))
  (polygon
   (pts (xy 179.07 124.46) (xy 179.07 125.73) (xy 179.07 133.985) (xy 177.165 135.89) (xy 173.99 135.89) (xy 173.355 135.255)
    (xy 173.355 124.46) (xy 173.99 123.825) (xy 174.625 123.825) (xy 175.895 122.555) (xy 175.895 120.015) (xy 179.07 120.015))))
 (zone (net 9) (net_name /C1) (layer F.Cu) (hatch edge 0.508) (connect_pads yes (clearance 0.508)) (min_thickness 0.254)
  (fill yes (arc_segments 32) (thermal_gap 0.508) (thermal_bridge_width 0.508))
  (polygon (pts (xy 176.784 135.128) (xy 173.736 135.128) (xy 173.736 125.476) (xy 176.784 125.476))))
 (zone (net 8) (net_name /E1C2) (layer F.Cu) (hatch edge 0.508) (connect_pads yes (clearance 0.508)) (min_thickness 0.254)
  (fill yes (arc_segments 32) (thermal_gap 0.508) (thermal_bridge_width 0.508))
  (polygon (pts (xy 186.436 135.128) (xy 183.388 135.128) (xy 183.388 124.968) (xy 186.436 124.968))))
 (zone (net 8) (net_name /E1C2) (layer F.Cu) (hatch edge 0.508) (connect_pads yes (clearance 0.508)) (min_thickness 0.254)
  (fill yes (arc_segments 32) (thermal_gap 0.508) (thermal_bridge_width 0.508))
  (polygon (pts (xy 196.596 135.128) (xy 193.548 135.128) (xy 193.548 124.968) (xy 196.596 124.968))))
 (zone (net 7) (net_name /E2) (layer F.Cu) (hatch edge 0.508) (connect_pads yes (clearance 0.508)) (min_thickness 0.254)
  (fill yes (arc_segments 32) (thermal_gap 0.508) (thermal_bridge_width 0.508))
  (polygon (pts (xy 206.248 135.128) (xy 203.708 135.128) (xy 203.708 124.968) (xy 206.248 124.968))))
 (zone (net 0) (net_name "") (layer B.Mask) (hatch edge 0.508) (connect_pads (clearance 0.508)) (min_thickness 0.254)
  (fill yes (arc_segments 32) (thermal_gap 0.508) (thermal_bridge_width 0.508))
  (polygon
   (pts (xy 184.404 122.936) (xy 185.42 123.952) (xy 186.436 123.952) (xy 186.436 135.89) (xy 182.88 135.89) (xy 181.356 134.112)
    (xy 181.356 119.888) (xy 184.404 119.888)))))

